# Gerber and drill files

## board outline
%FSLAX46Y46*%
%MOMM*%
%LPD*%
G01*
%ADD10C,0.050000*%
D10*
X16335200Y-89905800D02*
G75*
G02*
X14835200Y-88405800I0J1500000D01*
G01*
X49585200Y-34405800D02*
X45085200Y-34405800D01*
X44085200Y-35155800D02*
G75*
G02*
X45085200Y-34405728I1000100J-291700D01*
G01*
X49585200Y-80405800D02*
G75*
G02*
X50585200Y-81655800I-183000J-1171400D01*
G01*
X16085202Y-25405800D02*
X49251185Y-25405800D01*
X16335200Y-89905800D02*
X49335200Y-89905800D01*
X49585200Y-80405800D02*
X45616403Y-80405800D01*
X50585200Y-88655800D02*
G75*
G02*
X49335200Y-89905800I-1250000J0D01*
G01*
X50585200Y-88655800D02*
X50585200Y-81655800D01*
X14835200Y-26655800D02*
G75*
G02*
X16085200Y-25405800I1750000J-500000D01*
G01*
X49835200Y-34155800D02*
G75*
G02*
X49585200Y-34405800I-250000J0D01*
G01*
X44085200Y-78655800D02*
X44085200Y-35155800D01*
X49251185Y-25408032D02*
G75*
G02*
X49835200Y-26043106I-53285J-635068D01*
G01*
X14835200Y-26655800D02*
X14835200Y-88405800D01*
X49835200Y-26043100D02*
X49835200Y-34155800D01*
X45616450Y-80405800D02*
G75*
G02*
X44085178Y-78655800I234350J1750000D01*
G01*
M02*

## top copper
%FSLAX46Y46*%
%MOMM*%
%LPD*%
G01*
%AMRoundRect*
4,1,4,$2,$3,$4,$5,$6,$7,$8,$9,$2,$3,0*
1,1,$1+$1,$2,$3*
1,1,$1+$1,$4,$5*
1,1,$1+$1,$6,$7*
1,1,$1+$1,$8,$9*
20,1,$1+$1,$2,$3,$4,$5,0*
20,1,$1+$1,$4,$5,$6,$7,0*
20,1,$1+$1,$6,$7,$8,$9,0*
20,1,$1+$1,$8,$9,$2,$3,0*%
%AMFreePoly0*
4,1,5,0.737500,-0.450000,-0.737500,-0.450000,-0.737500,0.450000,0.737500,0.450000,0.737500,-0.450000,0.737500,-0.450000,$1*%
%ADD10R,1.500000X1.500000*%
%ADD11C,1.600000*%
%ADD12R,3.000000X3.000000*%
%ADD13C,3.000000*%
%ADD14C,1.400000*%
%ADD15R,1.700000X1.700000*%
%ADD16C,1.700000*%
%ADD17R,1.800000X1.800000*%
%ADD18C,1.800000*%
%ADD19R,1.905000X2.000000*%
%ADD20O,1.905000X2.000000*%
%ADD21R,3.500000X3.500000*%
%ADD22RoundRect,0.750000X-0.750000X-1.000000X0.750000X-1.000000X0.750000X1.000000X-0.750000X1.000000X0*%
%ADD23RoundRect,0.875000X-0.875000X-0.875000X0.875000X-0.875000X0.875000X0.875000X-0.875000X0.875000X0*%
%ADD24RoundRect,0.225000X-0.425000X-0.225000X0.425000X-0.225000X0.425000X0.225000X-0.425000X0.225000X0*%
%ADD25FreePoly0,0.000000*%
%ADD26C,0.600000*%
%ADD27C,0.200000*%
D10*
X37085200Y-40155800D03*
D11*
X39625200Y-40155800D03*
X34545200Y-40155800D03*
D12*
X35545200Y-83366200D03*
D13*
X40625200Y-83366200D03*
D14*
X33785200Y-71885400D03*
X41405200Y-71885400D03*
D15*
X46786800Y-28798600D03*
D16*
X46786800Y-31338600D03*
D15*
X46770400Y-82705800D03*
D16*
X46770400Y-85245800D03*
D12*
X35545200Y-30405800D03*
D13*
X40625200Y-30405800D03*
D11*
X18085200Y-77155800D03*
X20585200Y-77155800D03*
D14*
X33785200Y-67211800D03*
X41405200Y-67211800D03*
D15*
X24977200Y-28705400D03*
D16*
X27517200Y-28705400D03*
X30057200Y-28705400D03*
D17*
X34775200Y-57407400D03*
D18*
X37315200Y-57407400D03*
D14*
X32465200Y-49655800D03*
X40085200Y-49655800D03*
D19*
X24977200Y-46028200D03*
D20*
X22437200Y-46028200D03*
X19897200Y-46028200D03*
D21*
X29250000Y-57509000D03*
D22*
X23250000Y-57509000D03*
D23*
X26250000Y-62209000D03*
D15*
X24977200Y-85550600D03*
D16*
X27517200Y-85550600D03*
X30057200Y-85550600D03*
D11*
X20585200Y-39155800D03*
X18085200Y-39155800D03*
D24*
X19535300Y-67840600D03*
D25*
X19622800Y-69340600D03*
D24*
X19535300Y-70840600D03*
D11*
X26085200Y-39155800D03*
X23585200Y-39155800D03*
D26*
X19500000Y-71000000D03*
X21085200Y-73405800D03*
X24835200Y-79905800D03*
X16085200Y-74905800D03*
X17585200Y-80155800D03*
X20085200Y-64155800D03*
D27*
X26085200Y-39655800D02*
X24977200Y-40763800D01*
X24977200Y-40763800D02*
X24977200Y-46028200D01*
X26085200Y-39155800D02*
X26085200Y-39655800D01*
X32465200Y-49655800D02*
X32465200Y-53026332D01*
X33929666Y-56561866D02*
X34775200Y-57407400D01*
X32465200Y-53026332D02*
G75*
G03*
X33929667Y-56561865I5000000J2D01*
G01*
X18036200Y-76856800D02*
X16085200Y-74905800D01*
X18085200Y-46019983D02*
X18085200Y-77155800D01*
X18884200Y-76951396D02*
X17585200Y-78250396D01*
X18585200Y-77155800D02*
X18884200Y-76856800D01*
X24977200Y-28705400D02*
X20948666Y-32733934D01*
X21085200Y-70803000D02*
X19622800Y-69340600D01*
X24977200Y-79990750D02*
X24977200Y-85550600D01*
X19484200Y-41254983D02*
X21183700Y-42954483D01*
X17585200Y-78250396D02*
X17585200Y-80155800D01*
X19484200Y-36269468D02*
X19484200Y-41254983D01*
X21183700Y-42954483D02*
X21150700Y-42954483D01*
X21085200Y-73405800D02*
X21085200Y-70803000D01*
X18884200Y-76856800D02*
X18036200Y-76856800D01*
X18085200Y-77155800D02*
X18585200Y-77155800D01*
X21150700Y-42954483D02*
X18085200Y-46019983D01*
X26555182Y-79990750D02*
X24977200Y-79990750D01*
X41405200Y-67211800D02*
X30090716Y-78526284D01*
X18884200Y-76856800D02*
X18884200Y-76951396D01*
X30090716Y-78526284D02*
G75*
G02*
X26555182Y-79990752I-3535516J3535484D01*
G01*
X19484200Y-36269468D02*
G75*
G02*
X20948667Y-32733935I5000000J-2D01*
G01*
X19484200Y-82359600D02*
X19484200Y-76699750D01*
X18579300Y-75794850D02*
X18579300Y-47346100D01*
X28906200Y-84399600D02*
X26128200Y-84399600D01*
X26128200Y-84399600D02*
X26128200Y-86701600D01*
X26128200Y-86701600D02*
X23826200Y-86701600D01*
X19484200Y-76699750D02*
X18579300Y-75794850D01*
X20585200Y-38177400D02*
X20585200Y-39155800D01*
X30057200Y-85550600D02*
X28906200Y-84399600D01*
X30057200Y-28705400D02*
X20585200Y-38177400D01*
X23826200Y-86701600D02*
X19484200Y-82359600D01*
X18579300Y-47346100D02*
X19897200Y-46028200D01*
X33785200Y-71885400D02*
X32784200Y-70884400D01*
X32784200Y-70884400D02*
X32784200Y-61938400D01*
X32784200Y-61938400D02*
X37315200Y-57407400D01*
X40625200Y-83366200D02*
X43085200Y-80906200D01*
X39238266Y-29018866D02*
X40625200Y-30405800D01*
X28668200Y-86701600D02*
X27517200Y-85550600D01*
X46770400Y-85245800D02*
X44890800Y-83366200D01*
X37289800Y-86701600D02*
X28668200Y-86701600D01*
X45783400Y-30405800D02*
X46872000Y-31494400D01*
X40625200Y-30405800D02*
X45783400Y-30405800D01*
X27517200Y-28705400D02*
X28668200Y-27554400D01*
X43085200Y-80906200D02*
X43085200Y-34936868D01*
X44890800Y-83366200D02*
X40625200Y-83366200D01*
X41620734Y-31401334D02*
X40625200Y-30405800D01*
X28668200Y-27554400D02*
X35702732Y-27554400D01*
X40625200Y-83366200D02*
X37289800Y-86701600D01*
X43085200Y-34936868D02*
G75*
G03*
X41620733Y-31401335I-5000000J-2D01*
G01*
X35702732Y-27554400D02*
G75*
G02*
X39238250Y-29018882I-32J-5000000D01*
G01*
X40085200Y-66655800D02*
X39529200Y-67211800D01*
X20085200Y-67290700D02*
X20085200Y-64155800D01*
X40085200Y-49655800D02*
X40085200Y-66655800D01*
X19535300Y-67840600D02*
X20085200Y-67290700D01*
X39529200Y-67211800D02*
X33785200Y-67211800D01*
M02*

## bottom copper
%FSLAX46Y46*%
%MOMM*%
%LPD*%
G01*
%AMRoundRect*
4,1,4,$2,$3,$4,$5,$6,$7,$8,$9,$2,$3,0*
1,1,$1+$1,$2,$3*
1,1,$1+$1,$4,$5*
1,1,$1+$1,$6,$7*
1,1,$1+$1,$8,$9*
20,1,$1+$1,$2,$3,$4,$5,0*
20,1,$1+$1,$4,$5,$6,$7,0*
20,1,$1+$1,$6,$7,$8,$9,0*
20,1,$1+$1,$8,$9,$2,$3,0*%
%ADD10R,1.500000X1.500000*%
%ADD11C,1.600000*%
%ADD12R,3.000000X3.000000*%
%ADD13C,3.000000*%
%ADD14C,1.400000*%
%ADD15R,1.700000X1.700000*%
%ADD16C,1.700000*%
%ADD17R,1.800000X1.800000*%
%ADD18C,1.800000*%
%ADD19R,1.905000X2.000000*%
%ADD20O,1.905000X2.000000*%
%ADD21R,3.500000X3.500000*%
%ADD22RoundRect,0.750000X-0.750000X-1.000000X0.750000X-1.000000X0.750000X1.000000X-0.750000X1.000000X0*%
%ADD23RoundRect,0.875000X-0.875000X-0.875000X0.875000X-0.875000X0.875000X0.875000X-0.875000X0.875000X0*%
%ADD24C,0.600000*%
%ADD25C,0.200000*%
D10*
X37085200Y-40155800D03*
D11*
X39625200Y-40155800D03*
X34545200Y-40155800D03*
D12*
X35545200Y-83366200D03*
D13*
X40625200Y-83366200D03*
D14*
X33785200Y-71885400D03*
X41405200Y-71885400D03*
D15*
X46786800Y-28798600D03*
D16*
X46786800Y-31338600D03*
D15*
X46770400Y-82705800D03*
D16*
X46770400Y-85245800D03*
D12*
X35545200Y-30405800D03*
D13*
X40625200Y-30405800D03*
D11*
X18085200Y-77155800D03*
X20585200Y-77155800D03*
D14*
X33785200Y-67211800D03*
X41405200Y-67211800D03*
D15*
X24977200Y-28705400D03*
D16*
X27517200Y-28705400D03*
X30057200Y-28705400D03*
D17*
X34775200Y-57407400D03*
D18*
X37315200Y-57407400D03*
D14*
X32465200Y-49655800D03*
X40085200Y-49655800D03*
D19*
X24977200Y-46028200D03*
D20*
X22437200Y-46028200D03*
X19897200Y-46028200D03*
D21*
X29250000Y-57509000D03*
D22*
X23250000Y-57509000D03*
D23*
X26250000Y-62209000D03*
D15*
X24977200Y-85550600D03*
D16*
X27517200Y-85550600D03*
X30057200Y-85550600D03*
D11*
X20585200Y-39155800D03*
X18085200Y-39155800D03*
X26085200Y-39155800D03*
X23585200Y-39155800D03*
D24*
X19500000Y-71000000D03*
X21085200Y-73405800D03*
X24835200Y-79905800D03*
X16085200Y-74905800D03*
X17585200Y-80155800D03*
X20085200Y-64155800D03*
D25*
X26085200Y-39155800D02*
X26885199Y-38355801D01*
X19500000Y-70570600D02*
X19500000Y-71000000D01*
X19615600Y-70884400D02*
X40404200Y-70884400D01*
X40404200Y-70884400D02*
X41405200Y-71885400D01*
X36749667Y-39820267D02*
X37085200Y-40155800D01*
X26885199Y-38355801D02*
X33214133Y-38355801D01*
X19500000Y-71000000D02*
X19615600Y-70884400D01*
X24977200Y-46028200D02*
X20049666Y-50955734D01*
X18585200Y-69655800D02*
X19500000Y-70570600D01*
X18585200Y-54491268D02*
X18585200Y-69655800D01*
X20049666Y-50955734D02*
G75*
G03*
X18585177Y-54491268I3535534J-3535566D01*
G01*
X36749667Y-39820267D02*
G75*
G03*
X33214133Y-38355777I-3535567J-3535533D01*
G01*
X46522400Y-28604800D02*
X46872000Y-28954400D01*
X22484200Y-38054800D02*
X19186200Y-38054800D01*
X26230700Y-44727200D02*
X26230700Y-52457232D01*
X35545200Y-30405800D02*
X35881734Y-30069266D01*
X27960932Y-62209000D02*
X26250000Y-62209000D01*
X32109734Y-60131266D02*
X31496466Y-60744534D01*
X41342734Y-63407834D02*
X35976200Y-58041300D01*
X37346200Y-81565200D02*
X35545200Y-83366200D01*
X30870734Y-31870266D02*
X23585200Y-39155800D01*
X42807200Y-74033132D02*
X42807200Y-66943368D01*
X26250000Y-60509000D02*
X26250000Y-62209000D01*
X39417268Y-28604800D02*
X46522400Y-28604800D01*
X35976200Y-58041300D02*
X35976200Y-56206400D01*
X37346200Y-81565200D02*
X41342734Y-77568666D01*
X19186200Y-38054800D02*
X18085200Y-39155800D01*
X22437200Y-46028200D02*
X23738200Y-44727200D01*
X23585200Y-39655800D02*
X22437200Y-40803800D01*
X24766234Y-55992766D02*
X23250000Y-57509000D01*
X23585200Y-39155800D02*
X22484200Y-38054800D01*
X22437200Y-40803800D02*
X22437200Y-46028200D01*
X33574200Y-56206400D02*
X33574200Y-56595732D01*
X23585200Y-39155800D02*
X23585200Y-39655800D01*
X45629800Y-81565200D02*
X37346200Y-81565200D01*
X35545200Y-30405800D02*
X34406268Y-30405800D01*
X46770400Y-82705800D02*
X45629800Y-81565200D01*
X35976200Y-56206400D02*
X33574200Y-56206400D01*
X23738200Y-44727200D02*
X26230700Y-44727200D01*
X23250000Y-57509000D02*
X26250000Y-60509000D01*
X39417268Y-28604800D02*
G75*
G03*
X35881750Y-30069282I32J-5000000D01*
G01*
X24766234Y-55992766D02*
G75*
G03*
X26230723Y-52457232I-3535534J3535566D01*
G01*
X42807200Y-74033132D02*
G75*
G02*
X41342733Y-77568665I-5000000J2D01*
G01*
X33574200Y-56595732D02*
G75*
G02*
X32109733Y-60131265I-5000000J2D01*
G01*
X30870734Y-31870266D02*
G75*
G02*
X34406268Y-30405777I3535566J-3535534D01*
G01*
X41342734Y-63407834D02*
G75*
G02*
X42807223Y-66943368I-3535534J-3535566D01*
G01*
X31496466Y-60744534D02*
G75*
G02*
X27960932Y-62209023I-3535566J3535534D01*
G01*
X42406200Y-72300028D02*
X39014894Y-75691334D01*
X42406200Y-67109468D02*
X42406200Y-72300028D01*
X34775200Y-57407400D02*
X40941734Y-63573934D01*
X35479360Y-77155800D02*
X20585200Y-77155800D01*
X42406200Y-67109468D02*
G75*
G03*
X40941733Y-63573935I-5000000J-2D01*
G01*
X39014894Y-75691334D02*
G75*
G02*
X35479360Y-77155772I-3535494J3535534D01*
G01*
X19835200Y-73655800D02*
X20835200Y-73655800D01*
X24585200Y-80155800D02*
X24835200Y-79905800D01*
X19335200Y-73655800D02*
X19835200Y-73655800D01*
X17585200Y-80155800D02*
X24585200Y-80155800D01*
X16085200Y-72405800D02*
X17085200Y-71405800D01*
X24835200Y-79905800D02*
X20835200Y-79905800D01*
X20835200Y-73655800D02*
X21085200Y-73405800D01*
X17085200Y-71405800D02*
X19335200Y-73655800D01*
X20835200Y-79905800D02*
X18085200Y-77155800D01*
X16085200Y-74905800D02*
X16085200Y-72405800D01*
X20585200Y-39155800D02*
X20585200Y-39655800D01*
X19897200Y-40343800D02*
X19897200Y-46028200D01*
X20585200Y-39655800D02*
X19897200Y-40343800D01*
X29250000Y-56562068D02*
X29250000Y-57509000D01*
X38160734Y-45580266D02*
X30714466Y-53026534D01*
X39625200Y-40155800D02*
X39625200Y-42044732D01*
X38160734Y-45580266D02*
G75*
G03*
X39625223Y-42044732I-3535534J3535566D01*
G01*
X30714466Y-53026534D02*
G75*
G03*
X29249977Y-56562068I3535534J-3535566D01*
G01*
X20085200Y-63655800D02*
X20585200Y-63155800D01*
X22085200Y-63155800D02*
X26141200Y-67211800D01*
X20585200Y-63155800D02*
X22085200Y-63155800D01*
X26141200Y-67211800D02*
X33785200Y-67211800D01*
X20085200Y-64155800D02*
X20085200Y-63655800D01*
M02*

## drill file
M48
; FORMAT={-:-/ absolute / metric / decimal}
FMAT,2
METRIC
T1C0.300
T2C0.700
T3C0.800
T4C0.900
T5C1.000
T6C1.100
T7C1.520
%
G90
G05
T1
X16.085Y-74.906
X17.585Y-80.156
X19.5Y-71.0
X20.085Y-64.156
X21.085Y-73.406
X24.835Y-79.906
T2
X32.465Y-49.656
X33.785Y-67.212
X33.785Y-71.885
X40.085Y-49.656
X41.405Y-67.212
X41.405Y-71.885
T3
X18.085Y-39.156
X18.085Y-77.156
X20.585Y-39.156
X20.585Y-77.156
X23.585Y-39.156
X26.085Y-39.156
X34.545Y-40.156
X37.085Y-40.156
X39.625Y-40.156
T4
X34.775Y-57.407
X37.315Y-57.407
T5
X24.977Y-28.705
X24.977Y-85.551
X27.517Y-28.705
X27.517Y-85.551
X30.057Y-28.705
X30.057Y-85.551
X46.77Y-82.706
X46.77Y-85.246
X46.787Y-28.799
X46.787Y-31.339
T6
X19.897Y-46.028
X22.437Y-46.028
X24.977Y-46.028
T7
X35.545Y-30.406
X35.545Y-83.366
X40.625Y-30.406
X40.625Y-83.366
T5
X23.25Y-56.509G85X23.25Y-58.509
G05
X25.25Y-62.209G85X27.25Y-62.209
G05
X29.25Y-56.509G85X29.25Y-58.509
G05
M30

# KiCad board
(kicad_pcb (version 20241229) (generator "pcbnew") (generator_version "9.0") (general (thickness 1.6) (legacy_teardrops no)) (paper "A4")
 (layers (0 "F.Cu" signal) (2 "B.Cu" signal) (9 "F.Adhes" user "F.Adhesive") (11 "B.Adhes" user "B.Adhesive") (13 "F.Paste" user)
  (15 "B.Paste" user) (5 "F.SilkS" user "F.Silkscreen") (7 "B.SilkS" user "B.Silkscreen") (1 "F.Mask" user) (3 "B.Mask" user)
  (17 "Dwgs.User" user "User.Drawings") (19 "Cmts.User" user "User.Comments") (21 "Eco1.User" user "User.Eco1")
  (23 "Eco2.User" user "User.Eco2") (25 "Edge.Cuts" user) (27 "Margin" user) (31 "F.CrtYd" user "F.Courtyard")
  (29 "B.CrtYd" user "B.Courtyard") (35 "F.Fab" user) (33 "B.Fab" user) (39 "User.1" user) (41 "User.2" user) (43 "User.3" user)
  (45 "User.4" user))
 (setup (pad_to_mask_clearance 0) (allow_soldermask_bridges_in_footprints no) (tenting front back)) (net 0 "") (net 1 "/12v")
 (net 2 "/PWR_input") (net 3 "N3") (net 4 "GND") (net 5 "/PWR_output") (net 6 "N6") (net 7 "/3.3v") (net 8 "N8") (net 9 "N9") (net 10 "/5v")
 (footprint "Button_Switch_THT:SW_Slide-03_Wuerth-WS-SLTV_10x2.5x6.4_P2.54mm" (layer "F.Cu") (at 37.0852 40.1558 180)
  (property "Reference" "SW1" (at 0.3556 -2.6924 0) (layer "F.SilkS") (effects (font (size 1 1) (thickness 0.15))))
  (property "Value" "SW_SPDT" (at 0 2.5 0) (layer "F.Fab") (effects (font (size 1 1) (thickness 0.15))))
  (pad "1" thru_hole rect (at 0 0 180) (size 1.5 1.5) (drill 0.8) (layers "*.Cu" "*.Mask") (remove_unused_layers no) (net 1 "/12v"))
  (pad "2" thru_hole circle (at -2.54 0 180) (size 1.6 1.6) (drill 0.8) (layers "*.Cu" "*.Mask") (remove_unused_layers no)
   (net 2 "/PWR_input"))
  (pad "3" thru_hole circle (at 2.54 0 180) (size 1.6 1.6) (drill 0.8) (layers "*.Cu" "*.Mask") (remove_unused_layers no) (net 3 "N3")))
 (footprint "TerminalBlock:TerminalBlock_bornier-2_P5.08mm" (layer "F.Cu") (at 35.5452 83.3662)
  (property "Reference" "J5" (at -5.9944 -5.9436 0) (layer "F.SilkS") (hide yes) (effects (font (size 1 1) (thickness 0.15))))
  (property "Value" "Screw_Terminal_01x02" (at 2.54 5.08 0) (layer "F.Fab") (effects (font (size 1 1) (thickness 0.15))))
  (pad "1" thru_hole rect (at 0 0) (size 3 3) (drill 1.52) (layers "*.Cu" "*.Mask") (remove_unused_layers no) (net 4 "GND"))
  (pad "2" thru_hole circle (at 5.08 0) (size 3 3) (drill 1.52) (layers "*.Cu" "*.Mask") (remove_unused_layers no) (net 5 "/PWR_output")))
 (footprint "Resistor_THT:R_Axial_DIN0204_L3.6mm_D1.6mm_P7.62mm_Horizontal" (layer "F.Cu") (at 33.7852 71.8854)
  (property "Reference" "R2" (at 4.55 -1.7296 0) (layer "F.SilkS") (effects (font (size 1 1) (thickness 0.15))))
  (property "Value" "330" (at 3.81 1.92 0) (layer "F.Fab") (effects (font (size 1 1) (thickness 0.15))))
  (pad "1" thru_hole circle (at 0 0) (size 1.4 1.4) (drill 0.7) (layers "*.Cu" "*.Mask") (remove_unused_layers no) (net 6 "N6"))
  (pad "2" thru_hole circle (at 7.62 0) (size 1.4 1.4) (drill 0.7) (layers "*.Cu" "*.Mask") (remove_unused_layers no) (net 1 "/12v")))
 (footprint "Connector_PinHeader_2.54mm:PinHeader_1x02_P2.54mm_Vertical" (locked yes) (layer "F.Cu") (at 46.7868 28.7986)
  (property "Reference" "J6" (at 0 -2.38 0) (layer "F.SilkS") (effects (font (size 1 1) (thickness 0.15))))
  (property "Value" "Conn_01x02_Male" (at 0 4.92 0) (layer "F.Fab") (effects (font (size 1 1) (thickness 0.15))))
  (pad "1" thru_hole rect (at 0 0) (size 1.7 1.7) (drill 1) (layers "*.Cu" "*.Mask") (remove_unused_layers no) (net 4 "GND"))
  (pad "2" thru_hole circle (at 0 2.54) (size 1.7 1.7) (drill 1) (layers "*.Cu" "*.Mask") (remove_unused_layers no) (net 5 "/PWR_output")))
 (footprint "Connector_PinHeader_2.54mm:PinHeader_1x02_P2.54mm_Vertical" (layer "F.Cu") (at 46.7704 82.7058)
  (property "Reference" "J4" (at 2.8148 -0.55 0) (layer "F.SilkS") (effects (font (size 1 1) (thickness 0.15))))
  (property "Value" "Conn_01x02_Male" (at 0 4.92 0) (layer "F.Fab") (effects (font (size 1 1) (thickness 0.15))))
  (pad "1" thru_hole rect (at 0 0) (size 1.7 1.7) (drill 1) (layers "*.Cu" "*.Mask") (remove_unused_layers no) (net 4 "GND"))
  (pad "2" thru_hole circle (at 0 2.54) (size 1.7 1.7) (drill 1) (layers "*.Cu" "*.Mask") (remove_unused_layers no) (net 5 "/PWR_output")))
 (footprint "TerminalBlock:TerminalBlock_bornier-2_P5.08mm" (layer "F.Cu") (at 35.5452 30.4058)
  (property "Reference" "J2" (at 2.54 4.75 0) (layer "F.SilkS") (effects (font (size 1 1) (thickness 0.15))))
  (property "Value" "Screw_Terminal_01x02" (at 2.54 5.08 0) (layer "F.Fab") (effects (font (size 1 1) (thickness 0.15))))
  (pad "1" thru_hole rect (at 0 0) (size 3 3) (drill 1.52) (layers "*.Cu" "*.Mask") (remove_unused_layers no) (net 4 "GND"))
  (pad "2" thru_hole circle (at 5.08 0) (size 3 3) (drill 1.52) (layers "*.Cu" "*.Mask") (remove_unused_layers no) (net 5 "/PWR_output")))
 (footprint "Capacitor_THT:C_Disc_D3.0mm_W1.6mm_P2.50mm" (layer "F.Cu") (at 18.0852 77.1558)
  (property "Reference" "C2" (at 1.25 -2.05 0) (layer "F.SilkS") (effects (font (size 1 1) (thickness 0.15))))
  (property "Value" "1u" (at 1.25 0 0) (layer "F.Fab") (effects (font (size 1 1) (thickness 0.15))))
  (pad "1" thru_hole circle (at 0 0) (size 1.6 1.6) (drill 0.8) (layers "*.Cu" "*.Mask") (remove_unused_layers no) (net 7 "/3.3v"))
  (pad "2" thru_hole circle (at 2.5 0) (size 1.6 1.6) (drill 0.8) (layers "*.Cu" "*.Mask") (remove_unused_layers no) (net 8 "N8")))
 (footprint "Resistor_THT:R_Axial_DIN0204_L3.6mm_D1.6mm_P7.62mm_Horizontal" (layer "F.Cu") (at 33.7852 67.2118)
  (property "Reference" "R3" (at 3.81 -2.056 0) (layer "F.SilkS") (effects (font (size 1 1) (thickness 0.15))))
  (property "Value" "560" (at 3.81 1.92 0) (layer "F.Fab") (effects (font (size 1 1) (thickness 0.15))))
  (pad "1" thru_hole circle (at 0 0) (size 1.4 1.4) (drill 0.7) (layers "*.Cu" "*.Mask") (remove_unused_layers no) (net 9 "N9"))
  (pad "2" thru_hole circle (at 7.62 0) (size 1.4 1.4) (drill 0.7) (layers "*.Cu" "*.Mask") (remove_unused_layers no) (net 7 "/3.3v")))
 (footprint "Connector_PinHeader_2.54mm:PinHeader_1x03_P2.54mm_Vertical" (layer "F.Cu") (at 24.9772 28.7054 90)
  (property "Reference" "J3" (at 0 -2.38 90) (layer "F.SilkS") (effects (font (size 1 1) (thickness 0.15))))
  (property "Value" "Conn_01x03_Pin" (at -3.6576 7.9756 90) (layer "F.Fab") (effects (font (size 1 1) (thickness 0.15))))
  (pad "1" thru_hole rect (at 0 0 90) (size 1.7 1.7) (drill 1) (layers "*.Cu" "*.Mask") (remove_unused_layers no) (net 7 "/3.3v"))
  (pad "2" thru_hole circle (at 0 2.54 90) (size 1.7 1.7) (drill 1) (layers "*.Cu" "*.Mask") (remove_unused_layers no) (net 5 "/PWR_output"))
  (pad "3" thru_hole circle (at 0 5.08 90) (size 1.7 1.7) (drill 1) (layers "*.Cu" "*.Mask") (remove_unused_layers no) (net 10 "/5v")))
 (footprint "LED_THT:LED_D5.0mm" (layer "F.Cu") (at 34.7752 57.4074)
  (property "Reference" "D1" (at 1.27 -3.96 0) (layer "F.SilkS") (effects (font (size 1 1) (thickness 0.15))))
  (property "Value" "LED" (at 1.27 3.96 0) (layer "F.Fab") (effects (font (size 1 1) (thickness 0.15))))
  (pad "1" thru_hole rect (at 0 0) (size 1.8 1.8) (drill 0.9) (layers "*.Cu" "*.Mask") (remove_unused_layers no) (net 8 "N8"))
  (pad "2" thru_hole circle (at 2.54 0) (size 1.8 1.8) (drill 0.9) (layers "*.Cu" "*.Mask") (remove_unused_layers no) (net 6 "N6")))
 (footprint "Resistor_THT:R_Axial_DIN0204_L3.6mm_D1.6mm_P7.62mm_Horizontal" (layer "F.Cu") (at 32.4652 49.6558)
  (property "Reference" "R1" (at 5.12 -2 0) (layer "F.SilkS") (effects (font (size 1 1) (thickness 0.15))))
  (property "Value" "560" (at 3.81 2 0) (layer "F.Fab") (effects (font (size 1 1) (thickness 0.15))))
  (pad "1" thru_hole circle (at 0 0) (size 1.4 1.4) (drill 0.7) (layers "*.Cu" "*.Mask") (remove_unused_layers no) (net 8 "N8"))
  (pad "2" thru_hole circle (at 7.62 0) (size 1.4 1.4) (drill 0.7) (layers "*.Cu" "*.Mask") (remove_unused_layers no) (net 9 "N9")))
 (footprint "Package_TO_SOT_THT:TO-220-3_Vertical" (layer "F.Cu") (at 24.9772 46.0282 180)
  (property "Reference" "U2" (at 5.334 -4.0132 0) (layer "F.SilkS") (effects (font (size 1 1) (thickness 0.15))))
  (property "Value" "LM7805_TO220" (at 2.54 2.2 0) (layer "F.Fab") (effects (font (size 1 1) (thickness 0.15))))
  (pad "1" thru_hole rect (at 0 0 180) (size 1.905 2) (drill 1.1) (layers "*.Cu" "*.Mask") (remove_unused_layers no) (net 1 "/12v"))
  (pad "2" thru_hole oval (at 2.54 0 180) (size 1.905 2) (drill 1.1) (layers "*.Cu" "*.Mask") (remove_unused_layers no) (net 4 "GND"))
  (pad "3" thru_hole oval (at 5.08 0 180) (size 1.905 2) (drill 1.1) (layers "*.Cu" "*.Mask") (remove_unused_layers no) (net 10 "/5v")))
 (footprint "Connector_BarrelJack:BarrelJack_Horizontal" (layer "F.Cu") (at 29.25 57.509)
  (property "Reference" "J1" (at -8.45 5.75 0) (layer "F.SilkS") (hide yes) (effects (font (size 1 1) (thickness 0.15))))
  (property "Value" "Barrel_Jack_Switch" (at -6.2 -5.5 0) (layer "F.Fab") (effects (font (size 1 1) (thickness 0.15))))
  (pad "1" thru_hole rect (at 0 0) (size 3.5 3.5) (drill oval 1 3) (layers "*.Cu" "*.Mask") (remove_unused_layers no) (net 2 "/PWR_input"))
  (pad "2" thru_hole roundrect (at -6 0) (size 3 3.5) (drill oval 1 3) (layers "*.Cu" "*.Mask") (remove_unused_layers no)
   (roundrect_rratio 0.25) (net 4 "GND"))
  (pad "3" thru_hole roundrect (at -3 4.7) (size 3.5 3.5) (drill oval 3 1) (layers "*.Cu" "*.Mask") (remove_unused_layers no)
   (roundrect_rratio 0.25) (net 4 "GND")))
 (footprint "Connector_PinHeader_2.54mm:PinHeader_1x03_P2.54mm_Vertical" (layer "F.Cu") (at 24.9772 85.5506 90)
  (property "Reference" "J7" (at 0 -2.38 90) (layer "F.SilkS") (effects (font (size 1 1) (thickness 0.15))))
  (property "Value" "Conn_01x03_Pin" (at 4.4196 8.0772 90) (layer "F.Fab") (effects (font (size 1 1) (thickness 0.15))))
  (pad "1" thru_hole rect (at 0 0 90) (size 1.7 1.7) (drill 1) (layers "*.Cu" "*.Mask") (remove_unused_layers no) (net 7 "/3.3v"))
  (pad "2" thru_hole circle (at 0 2.54 90) (size 1.7 1.7) (drill 1) (layers "*.Cu" "*.Mask") (remove_unused_layers no) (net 5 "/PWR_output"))
  (pad "3" thru_hole circle (at 0 5.08 90) (size 1.7 1.7) (drill 1) (layers "*.Cu" "*.Mask") (remove_unused_layers no) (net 10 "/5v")))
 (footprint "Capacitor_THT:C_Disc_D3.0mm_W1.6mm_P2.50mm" (layer "F.Cu") (at 20.5852 39.1558 180)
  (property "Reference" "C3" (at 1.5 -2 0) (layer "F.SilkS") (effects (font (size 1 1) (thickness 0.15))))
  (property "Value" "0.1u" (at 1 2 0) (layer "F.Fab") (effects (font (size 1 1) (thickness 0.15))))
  (pad "1" thru_hole circle (at 0 0 180) (size 1.6 1.6) (drill 0.8) (layers "*.Cu" "*.Mask") (remove_unused_layers no) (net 10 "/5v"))
  (pad "2" thru_hole circle (at 2.5 0 180) (size 1.6 1.6) (drill 0.8) (layers "*.Cu" "*.Mask") (remove_unused_layers no) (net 4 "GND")))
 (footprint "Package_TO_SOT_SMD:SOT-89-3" (layer "F.Cu") (at 21.4853 69.3406)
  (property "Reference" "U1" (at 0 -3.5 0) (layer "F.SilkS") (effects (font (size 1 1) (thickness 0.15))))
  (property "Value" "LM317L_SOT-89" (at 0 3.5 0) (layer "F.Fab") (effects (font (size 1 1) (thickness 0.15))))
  (pad "1" smd roundrect (at -1.95 -1.5) (size 1.3 0.9) (layers "F.Cu" "F.Mask" "F.Paste") (roundrect_rratio 0.25) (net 9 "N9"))
  (pad "2" smd custom (at -1.8625 0) (size 1.475 0.9) (layers "F.Cu" "F.Mask" "F.Paste") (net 7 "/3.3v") (zone_connect 2)
   (thermal_bridge_angle 45) (options (clearance outline) (anchor rect)) (primitives))
  (pad "3" smd roundrect (at -1.95 1.5) (size 1.3 0.9) (layers "F.Cu" "F.Mask" "F.Paste") (roundrect_rratio 0.25) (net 1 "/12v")))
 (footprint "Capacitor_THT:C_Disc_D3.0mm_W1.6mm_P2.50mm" (layer "F.Cu") (at 26.0852 39.1558 180)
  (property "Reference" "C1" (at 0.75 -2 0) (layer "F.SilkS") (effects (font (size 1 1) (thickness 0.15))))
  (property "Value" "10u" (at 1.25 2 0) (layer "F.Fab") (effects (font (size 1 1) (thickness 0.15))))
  (pad "1" thru_hole circle (at 0 0 180) (size 1.6 1.6) (drill 0.8) (layers "*.Cu" "*.Mask") (remove_unused_layers no) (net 1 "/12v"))
  (pad "2" thru_hole circle (at 2.5 0 180) (size 1.6 1.6) (drill 0.8) (layers "*.Cu" "*.Mask") (remove_unused_layers no) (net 4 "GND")))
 (gr_arc (start 16.3352 89.9058) (mid 15.27454 89.46646) (end 14.8352 88.4058) (stroke (width 0.05) (type default)) (layer "Edge.Cuts"))
 (gr_line (start 49.5852 34.4058) (end 45.0852 34.4058) (stroke (width 0.05) (type default)) (layer "Edge.Cuts"))
 (gr_arc (start 44.0852 35.1558) (mid 44.460207 34.61415) (end 45.0852 34.4058) (stroke (width 0.05) (type default)) (layer "Edge.Cuts"))
 (gr_arc (start 49.5852 80.4058) (mid 50.328016 80.836547) (end 50.5852 81.6558) (stroke (width 0.05) (type default)) (layer "Edge.Cuts"))
 (gr_line (start 16.085202 25.4058) (end 49.251185 25.4058) (stroke (width 0.05) (type default)) (layer "Edge.Cuts"))
 (gr_line (start 16.3352 89.9058) (end 49.3352 89.9058) (stroke (width 0.05) (type default)) (layer "Edge.Cuts"))
 (gr_line (start 49.5852 80.4058) (end 45.616403 80.4058) (stroke (width 0.05) (type default)) (layer "Edge.Cuts"))
 (gr_arc (start 50.5852 88.6558) (mid 50.219083 89.539683) (end 49.3352 89.9058) (stroke (width 0.05) (type default)) (layer "Edge.Cuts"))
 (gr_line (start 50.5852 88.6558) (end 50.5852 81.6558) (stroke (width 0.05) (type default)) (layer "Edge.Cuts"))
 (gr_arc (start 14.8352 26.6558) (mid 15.298246 25.868846) (end 16.0852 25.4058) (stroke (width 0.05) (type default)) (layer "Edge.Cuts"))
 (gr_arc (start 49.8352 34.1558) (mid 49.761977 34.332577) (end 49.5852 34.4058) (stroke (width 0.05) (type default)) (layer "Edge.Cuts"))
 (gr_line (start 44.0852 78.6558) (end 44.0852 35.1558) (stroke (width 0.05) (type default)) (layer "Edge.Cuts"))
 (gr_arc (start 49.251185 25.408032) (mid 49.667 25.611715) (end 49.8352 26.043106) (stroke (width 0.05) (type default)) (layer "Edge.Cuts"))
 (gr_line (start 14.8352 26.6558) (end 14.8352 88.4058) (stroke (width 0.05) (type default)) (layer "Edge.Cuts"))
 (gr_line (start 49.8352 26.0431) (end 49.8352 34.1558) (stroke (width 0.05) (type default)) (layer "Edge.Cuts"))
 (gr_arc (start 45.61645 80.4058) (mid 44.522057 79.818472) (end 44.0852 78.6558) (stroke (width 0.05) (type default)) (layer "Edge.Cuts"))
 (segment (start 26.0852 39.6558) (end 24.9772 40.7638) (width 0.2) (layer "F.Cu") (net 1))
 (segment (start 24.9772 40.7638) (end 24.9772 46.0282) (width 0.2) (layer "F.Cu") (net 1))
 (segment (start 26.0852 39.1558) (end 26.0852 39.6558) (width 0.2) (layer "F.Cu") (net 1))
 (via (at 19.5 71) (size 0.6) (drill 0.3) (layers "F.Cu" "B.Cu") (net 1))
 (segment (start 26.0852 39.1558) (end 26.885199 38.355801) (width 0.2) (layer "B.Cu") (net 1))
 (segment (start 19.5 70.5706) (end 19.5 71) (width 0.2) (layer "B.Cu") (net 1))
 (segment (start 19.6156 70.8844) (end 40.4042 70.8844) (width 0.2) (layer "B.Cu") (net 1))
 (segment (start 40.4042 70.8844) (end 41.4052 71.8854) (width 0.2) (layer "B.Cu") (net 1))
 (segment (start 36.749667 39.820267) (end 37.0852 40.1558) (width 0.2) (layer "B.Cu") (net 1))
 (segment (start 26.885199 38.355801) (end 33.214133 38.355801) (width 0.2) (layer "B.Cu") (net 1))
 (segment (start 19.5 71) (end 19.6156 70.8844) (width 0.2) (layer "B.Cu") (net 1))
 (segment (start 24.9772 46.0282) (end 20.049666 50.955734) (width 0.2) (layer "B.Cu") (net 1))
 (segment (start 18.5852 69.6558) (end 19.5 70.5706) (width 0.2) (layer "B.Cu") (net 1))
 (segment (start 18.5852 54.491268) (end 18.5852 69.6558) (width 0.2) (layer "B.Cu") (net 1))
 (arc (start 20.049666 50.955734) (mid 18.965802 52.577851) (end 18.5852 54.491268) (width 0.2) (layer "B.Cu") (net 1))
 (arc (start 36.749667 39.820267) (mid 35.12755 38.736403) (end 33.214133 38.355801) (width 0.2) (layer "B.Cu") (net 1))
 (segment (start 46.5224 28.6048) (end 46.872 28.9544) (width 0.2) (layer "B.Cu") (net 4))
 (segment (start 22.4842 38.0548) (end 19.1862 38.0548) (width 0.2) (layer "B.Cu") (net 4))
 (segment (start 26.2307 44.7272) (end 26.2307 52.457232) (width 0.2) (layer "B.Cu") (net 4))
 (segment (start 35.5452 30.4058) (end 35.881734 30.069266) (width 0.2) (layer "B.Cu") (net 4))
 (segment (start 27.960932 62.209) (end 26.25 62.209) (width 0.2) (layer "B.Cu") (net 4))
 (segment (start 32.109734 60.131266) (end 31.496466 60.744534) (width 0.2) (layer "B.Cu") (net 4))
 (segment (start 41.342734 63.407834) (end 35.9762 58.0413) (width 0.2) (layer "B.Cu") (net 4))
 (segment (start 37.3462 81.5652) (end 35.5452 83.3662) (width 0.2) (layer "B.Cu") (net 4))
 (segment (start 30.870734 31.870266) (end 23.5852 39.1558) (width 0.2) (layer "B.Cu") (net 4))
 (segment (start 42.8072 74.033132) (end 42.8072 66.943368) (width 0.2) (layer "B.Cu") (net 4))
 (segment (start 26.25 60.509) (end 26.25 62.209) (width 0.2) (layer "B.Cu") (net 4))
 (segment (start 39.417268 28.6048) (end 46.5224 28.6048) (width 0.2) (layer "B.Cu") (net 4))
 (segment (start 35.9762 58.0413) (end 35.9762 56.2064) (width 0.2) (layer "B.Cu") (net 4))
 (segment (start 37.3462 81.5652) (end 41.342734 77.568666) (width 0.2) (layer "B.Cu") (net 4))
 (segment (start 19.1862 38.0548) (end 18.0852 39.1558) (width 0.2) (layer "B.Cu") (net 4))
 (segment (start 22.4372 46.0282) (end 23.7382 44.7272) (width 0.2) (layer "B.Cu") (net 4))
 (segment (start 23.5852 39.6558) (end 22.4372 40.8038) (width 0.2) (layer "B.Cu") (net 4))
 (segment (start 24.766234 55.992766) (end 23.25 57.509) (width 0.2) (layer "B.Cu") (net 4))
 (segment (start 23.5852 39.1558) (end 22.4842 38.0548) (width 0.2) (layer "B.Cu") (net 4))
 (segment (start 22.4372 40.8038) (end 22.4372 46.0282) (width 0.2) (layer "B.Cu") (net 4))
 (segment (start 33.5742 56.2064) (end 33.5742 56.595732) (width 0.2) (layer "B.Cu") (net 4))
 (segment (start 23.5852 39.1558) (end 23.5852 39.6558) (width 0.2) (layer "B.Cu") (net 4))
 (segment (start 45.6298 81.5652) (end 37.3462 81.5652) (width 0.2) (layer "B.Cu") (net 4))
 (segment (start 35.5452 30.4058) (end 34.406268 30.4058) (width 0.2) (layer "B.Cu") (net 4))
 (segment (start 46.7704 82.7058) (end 45.6298 81.5652) (width 0.2) (layer "B.Cu") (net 4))
 (segment (start 35.9762 56.2064) (end 33.5742 56.2064) (width 0.2) (layer "B.Cu") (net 4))
 (segment (start 23.7382 44.7272) (end 26.2307 44.7272) (width 0.2) (layer "B.Cu") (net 4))
 (segment (start 23.25 57.509) (end 26.25 60.509) (width 0.2) (layer "B.Cu") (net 4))
 (arc (start 39.417268 28.6048) (mid 37.503851 28.985402) (end 35.881734 30.069266) (width 0.2) (layer "B.Cu") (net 4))
 (arc (start 24.766234 55.992766) (mid 25.850098 54.370649) (end 26.2307 52.457232) (width 0.2) (layer "B.Cu") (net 4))
 (arc (start 42.8072 74.033132) (mid 42.426598 75.946549) (end 41.342734 77.568666) (width 0.2) (layer "B.Cu") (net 4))
 (arc (start 33.5742 56.595732) (mid 33.193598 58.509149) (end 32.109734 60.131266) (width 0.2) (layer "B.Cu") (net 4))
 (arc (start 30.870734 31.870266) (mid 32.492851 30.786402) (end 34.406268 30.4058) (width 0.2) (layer "B.Cu") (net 4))
 (arc (start 41.342734 63.407834) (mid 42.426598 65.029951) (end 42.8072 66.943368) (width 0.2) (layer "B.Cu") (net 4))
 (arc (start 31.496466 60.744534) (mid 29.874349 61.828398) (end 27.960932 62.209) (width 0.2) (layer "B.Cu") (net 4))
 (segment (start 32.4652 49.6558) (end 32.4652 53.026332) (width 0.2) (layer "F.Cu") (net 8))
 (segment (start 33.929666 56.561866) (end 34.7752 57.4074) (width 0.2) (layer "F.Cu") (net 8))
 (arc (start 32.4652 53.026332) (mid 32.845802 54.939749) (end 33.929666 56.561866) (width 0.2) (layer "F.Cu") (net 8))
 (segment (start 42.4062 72.300028) (end 39.014894 75.691334) (width 0.2) (layer "B.Cu") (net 8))
 (segment (start 42.4062 67.109468) (end 42.4062 72.300028) (width 0.2) (layer "B.Cu") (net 8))
 (segment (start 34.7752 57.4074) (end 40.941734 63.573934) (width 0.2) (layer "B.Cu") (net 8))
 (segment (start 35.47936 77.1558) (end 20.5852 77.1558) (width 0.2) (layer "B.Cu") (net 8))
 (arc (start 42.4062 67.109468) (mid 42.025598 65.196051) (end 40.941734 63.573934) (width 0.2) (layer "B.Cu") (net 8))
 (arc (start 39.014894 75.691334) (mid 37.392777 76.775198) (end 35.47936 77.1558) (width 0.2) (layer "B.Cu") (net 8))
 (segment (start 18.0362 76.8568) (end 16.0852 74.9058) (width 0.2) (layer "F.Cu") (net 7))
 (segment (start 18.0852 46.019983) (end 18.0852 77.1558) (width 0.2) (layer "F.Cu") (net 7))
 (segment (start 18.8842 76.951396) (end 17.5852 78.250396) (width 0.2) (layer "F.Cu") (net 7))
 (segment (start 18.5852 77.1558) (end 18.8842 76.8568) (width 0.2) (layer "F.Cu") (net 7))
 (segment (start 24.9772 28.7054) (end 20.948666 32.733934) (width 0.2) (layer "F.Cu") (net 7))
 (segment (start 21.0852 70.803) (end 19.6228 69.3406) (width 0.2) (layer "F.Cu") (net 7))
 (segment (start 24.9772 79.99075) (end 24.9772 85.5506) (width 0.2) (layer "F.Cu") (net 7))
 (segment (start 19.4842 41.254983) (end 21.1837 42.954483) (width 0.2) (layer "F.Cu") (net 7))
 (segment (start 17.5852 78.250396) (end 17.5852 80.1558) (width 0.2) (layer "F.Cu") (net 7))
 (segment (start 19.4842 36.269468) (end 19.4842 41.254983) (width 0.2) (layer "F.Cu") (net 7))
 (segment (start 21.1837 42.954483) (end 21.1507 42.954483) (width 0.2) (layer "F.Cu") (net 7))
 (segment (start 21.0852 73.4058) (end 21.0852 70.803) (width 0.2) (layer "F.Cu") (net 7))
 (segment (start 18.8842 76.8568) (end 18.0362 76.8568) (width 0.2) (layer "F.Cu") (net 7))
 (segment (start 18.0852 77.1558) (end 18.5852 77.1558) (width 0.2) (layer "F.Cu") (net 7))
 (segment (start 21.1507 42.954483) (end 18.0852 46.019983) (width 0.2) (layer "F.Cu") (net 7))
 (segment (start 26.555182 79.99075) (end 24.9772 79.99075) (width 0.2) (layer "F.Cu") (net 7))
 (segment (start 41.4052 67.2118) (end 30.090716 78.526284) (width 0.2) (layer "F.Cu") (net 7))
 (segment (start 18.8842 76.8568) (end 18.8842 76.951396) (width 0.2) (layer "F.Cu") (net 7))
 (via (at 21.0852 73.4058) (size 0.6) (drill 0.3) (layers "F.Cu" "B.Cu") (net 7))
 (via (at 24.8352 79.9058) (size 0.6) (drill 0.3) (layers "F.Cu" "B.Cu") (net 7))
 (via (at 16.0852 74.9058) (size 0.6) (drill 0.3) (layers "F.Cu" "B.Cu") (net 7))
 (via (at 17.5852 80.1558) (size 0.6) (drill 0.3) (layers "F.Cu" "B.Cu") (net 7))
 (arc (start 30.090716 78.526284) (mid 28.468599 79.610148) (end 26.555182 79.99075) (width 0.2) (layer "F.Cu") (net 7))
 (arc (start 19.4842 36.269468) (mid 19.864802 34.356051) (end 20.948666 32.733934) (width 0.2) (layer "F.Cu") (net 7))
 (segment (start 19.8352 73.6558) (end 20.8352 73.6558) (width 0.2) (layer "B.Cu") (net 7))
 (segment (start 24.5852 80.1558) (end 24.8352 79.9058) (width 0.2) (layer "B.Cu") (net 7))
 (segment (start 19.3352 73.6558) (end 19.8352 73.6558) (width 0.2) (layer "B.Cu") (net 7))
 (segment (start 17.5852 80.1558) (end 24.5852 80.1558) (width 0.2) (layer "B.Cu") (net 7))
 (segment (start 16.0852 72.4058) (end 17.0852 71.4058) (width 0.2) (layer "B.Cu") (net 7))
 (segment (start 24.8352 79.9058) (end 20.8352 79.9058) (width 0.2) (layer "B.Cu") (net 7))
 (segment (start 20.8352 73.6558) (end 21.0852 73.4058) (width 0.2) (layer "B.Cu") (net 7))
 (segment (start 17.0852 71.4058) (end 19.3352 73.6558) (width 0.2) (layer "B.Cu") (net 7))
 (segment (start 20.8352 79.9058) (end 18.0852 77.1558) (width 0.2) (layer "B.Cu") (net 7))
 (segment (start 16.0852 74.9058) (end 16.0852 72.4058) (width 0.2) (layer "B.Cu") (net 7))
 (segment (start 19.4842 82.3596) (end 19.4842 76.69975) (width 0.2) (layer "F.Cu") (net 10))
 (segment (start 18.5793 75.79485) (end 18.5793 47.3461) (width 0.2) (layer "F.Cu") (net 10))
 (segment (start 28.9062 84.3996) (end 26.1282 84.3996) (width 0.2) (layer "F.Cu") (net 10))
 (segment (start 26.1282 84.3996) (end 26.1282 86.7016) (width 0.2) (layer "F.Cu") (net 10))
 (segment (start 26.1282 86.7016) (end 23.8262 86.7016) (width 0.2) (layer "F.Cu") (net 10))
 (segment (start 19.4842 76.69975) (end 18.5793 75.79485) (width 0.2) (layer "F.Cu") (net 10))
 (segment (start 20.5852 38.1774) (end 20.5852 39.1558) (width 0.2) (layer "F.Cu") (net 10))
 (segment (start 30.0572 85.5506) (end 28.9062 84.3996) (width 0.2) (layer "F.Cu") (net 10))
 (segment (start 30.0572 28.7054) (end 20.5852 38.1774) (width 0.2) (layer "F.Cu") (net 10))
 (segment (start 23.8262 86.7016) (end 19.4842 82.3596) (width 0.2) (layer "F.Cu") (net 10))
 (segment (start 18.5793 47.3461) (end 19.8972 46.0282) (width 0.2) (layer "F.Cu") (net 10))
 (segment (start 20.5852 39.1558) (end 20.5852 39.6558) (width 0.2) (layer "B.Cu") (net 10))
 (segment (start 19.8972 40.3438) (end 19.8972 46.0282) (width 0.2) (layer "B.Cu") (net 10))
 (segment (start 20.5852 39.6558) (end 19.8972 40.3438) (width 0.2) (layer "B.Cu") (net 10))
 (segment (start 33.7852 71.8854) (end 32.7842 70.8844) (width 0.2) (layer "F.Cu") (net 6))
 (segment (start 32.7842 70.8844) (end 32.7842 61.9384) (width 0.2) (layer "F.Cu") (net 6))
 (segment (start 32.7842 61.9384) (end 37.3152 57.4074) (width 0.2) (layer "F.Cu") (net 6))
 (segment (start 29.25 56.562068) (end 29.25 57.509) (width 0.2) (layer "B.Cu") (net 2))
 (segment (start 38.160734 45.580266) (end 30.714466 53.026534) (width 0.2) (layer "B.Cu") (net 2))
 (segment (start 39.6252 40.1558) (end 39.6252 42.044732) (width 0.2) (layer "B.Cu") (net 2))
 (arc (start 38.160734 45.580266) (mid 39.244598 43.958149) (end 39.6252 42.044732) (width 0.2) (layer "B.Cu") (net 2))
 (arc (start 30.714466 53.026534) (mid 29.630602 54.648651) (end 29.25 56.562068) (width 0.2) (layer "B.Cu") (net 2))
 (segment (start 40.6252 83.3662) (end 43.0852 80.9062) (width 0.2) (layer "F.Cu") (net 5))
 (segment (start 39.238266 29.018866) (end 40.6252 30.4058) (width 0.2) (layer "F.Cu") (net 5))
 (segment (start 28.6682 86.7016) (end 27.5172 85.5506) (width 0.2) (layer "F.Cu") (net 5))
 (segment (start 46.7704 85.2458) (end 44.8908 83.3662) (width 0.2) (layer "F.Cu") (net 5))
 (segment (start 37.2898 86.7016) (end 28.6682 86.7016) (width 0.2) (layer "F.Cu") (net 5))
 (segment (start 45.7834 30.4058) (end 46.872 31.4944) (width 0.2) (layer "F.Cu") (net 5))
 (segment (start 40.6252 30.4058) (end 45.7834 30.4058) (width 0.2) (layer "F.Cu") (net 5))
 (segment (start 27.5172 28.7054) (end 28.6682 27.5544) (width 0.2) (layer "F.Cu") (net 5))
 (segment (start 43.0852 80.9062) (end 43.0852 34.936868) (width 0.2) (layer "F.Cu") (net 5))
 (segment (start 44.8908 83.3662) (end 40.6252 83.3662) (width 0.2) (layer "F.Cu") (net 5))
 (segment (start 41.620734 31.401334) (end 40.6252 30.4058) (width 0.2) (layer "F.Cu") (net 5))
 (segment (start 28.6682 27.5544) (end 35.702732 27.5544) (width 0.2) (layer "F.Cu") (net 5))
 (segment (start 40.6252 83.3662) (end 37.2898 86.7016) (width 0.2) (layer "F.Cu") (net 5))
 (arc (start 43.0852 34.936868) (mid 42.704598 33.023451) (end 41.620734 31.401334) (width 0.2) (layer "F.Cu") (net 5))
 (arc (start 35.702732 27.5544) (mid 37.616149 27.935002) (end 39.238266 29.018866) (width 0.2) (layer "F.Cu") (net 5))
 (segment (start 40.0852 66.6558) (end 39.5292 67.2118) (width 0.2) (layer "F.Cu") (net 9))
 (segment (start 20.0852 67.2907) (end 20.0852 64.1558) (width 0.2) (layer "F.Cu") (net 9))
 (segment (start 40.0852 49.6558) (end 40.0852 66.6558) (width 0.2) (layer "F.Cu") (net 9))
 (segment (start 19.5353 67.8406) (end 20.0852 67.2907) (width 0.2) (layer "F.Cu") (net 9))
 (segment (start 39.5292 67.2118) (end 33.7852 67.2118) (width 0.2) (layer "F.Cu") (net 9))
 (via (at 20.0852 64.1558) (size 0.6) (drill 0.3) (layers "F.Cu" "B.Cu") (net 9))
 (segment (start 20.0852 63.6558) (end 20.5852 63.1558) (width 0.2) (layer "B.Cu") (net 9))
 (segment (start 22.0852 63.1558) (end 26.1412 67.2118) (width 0.2) (layer "B.Cu") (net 9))
 (segment (start 20.5852 63.1558) (end 22.0852 63.1558) (width 0.2) (layer "B.Cu") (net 9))
 (segment (start 26.1412 67.2118) (end 33.7852 67.2118) (width 0.2) (layer "B.Cu") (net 9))
 (segment (start 20.0852 64.1558) (end 20.0852 63.6558) (width 0.2) (layer "B.Cu") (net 9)))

